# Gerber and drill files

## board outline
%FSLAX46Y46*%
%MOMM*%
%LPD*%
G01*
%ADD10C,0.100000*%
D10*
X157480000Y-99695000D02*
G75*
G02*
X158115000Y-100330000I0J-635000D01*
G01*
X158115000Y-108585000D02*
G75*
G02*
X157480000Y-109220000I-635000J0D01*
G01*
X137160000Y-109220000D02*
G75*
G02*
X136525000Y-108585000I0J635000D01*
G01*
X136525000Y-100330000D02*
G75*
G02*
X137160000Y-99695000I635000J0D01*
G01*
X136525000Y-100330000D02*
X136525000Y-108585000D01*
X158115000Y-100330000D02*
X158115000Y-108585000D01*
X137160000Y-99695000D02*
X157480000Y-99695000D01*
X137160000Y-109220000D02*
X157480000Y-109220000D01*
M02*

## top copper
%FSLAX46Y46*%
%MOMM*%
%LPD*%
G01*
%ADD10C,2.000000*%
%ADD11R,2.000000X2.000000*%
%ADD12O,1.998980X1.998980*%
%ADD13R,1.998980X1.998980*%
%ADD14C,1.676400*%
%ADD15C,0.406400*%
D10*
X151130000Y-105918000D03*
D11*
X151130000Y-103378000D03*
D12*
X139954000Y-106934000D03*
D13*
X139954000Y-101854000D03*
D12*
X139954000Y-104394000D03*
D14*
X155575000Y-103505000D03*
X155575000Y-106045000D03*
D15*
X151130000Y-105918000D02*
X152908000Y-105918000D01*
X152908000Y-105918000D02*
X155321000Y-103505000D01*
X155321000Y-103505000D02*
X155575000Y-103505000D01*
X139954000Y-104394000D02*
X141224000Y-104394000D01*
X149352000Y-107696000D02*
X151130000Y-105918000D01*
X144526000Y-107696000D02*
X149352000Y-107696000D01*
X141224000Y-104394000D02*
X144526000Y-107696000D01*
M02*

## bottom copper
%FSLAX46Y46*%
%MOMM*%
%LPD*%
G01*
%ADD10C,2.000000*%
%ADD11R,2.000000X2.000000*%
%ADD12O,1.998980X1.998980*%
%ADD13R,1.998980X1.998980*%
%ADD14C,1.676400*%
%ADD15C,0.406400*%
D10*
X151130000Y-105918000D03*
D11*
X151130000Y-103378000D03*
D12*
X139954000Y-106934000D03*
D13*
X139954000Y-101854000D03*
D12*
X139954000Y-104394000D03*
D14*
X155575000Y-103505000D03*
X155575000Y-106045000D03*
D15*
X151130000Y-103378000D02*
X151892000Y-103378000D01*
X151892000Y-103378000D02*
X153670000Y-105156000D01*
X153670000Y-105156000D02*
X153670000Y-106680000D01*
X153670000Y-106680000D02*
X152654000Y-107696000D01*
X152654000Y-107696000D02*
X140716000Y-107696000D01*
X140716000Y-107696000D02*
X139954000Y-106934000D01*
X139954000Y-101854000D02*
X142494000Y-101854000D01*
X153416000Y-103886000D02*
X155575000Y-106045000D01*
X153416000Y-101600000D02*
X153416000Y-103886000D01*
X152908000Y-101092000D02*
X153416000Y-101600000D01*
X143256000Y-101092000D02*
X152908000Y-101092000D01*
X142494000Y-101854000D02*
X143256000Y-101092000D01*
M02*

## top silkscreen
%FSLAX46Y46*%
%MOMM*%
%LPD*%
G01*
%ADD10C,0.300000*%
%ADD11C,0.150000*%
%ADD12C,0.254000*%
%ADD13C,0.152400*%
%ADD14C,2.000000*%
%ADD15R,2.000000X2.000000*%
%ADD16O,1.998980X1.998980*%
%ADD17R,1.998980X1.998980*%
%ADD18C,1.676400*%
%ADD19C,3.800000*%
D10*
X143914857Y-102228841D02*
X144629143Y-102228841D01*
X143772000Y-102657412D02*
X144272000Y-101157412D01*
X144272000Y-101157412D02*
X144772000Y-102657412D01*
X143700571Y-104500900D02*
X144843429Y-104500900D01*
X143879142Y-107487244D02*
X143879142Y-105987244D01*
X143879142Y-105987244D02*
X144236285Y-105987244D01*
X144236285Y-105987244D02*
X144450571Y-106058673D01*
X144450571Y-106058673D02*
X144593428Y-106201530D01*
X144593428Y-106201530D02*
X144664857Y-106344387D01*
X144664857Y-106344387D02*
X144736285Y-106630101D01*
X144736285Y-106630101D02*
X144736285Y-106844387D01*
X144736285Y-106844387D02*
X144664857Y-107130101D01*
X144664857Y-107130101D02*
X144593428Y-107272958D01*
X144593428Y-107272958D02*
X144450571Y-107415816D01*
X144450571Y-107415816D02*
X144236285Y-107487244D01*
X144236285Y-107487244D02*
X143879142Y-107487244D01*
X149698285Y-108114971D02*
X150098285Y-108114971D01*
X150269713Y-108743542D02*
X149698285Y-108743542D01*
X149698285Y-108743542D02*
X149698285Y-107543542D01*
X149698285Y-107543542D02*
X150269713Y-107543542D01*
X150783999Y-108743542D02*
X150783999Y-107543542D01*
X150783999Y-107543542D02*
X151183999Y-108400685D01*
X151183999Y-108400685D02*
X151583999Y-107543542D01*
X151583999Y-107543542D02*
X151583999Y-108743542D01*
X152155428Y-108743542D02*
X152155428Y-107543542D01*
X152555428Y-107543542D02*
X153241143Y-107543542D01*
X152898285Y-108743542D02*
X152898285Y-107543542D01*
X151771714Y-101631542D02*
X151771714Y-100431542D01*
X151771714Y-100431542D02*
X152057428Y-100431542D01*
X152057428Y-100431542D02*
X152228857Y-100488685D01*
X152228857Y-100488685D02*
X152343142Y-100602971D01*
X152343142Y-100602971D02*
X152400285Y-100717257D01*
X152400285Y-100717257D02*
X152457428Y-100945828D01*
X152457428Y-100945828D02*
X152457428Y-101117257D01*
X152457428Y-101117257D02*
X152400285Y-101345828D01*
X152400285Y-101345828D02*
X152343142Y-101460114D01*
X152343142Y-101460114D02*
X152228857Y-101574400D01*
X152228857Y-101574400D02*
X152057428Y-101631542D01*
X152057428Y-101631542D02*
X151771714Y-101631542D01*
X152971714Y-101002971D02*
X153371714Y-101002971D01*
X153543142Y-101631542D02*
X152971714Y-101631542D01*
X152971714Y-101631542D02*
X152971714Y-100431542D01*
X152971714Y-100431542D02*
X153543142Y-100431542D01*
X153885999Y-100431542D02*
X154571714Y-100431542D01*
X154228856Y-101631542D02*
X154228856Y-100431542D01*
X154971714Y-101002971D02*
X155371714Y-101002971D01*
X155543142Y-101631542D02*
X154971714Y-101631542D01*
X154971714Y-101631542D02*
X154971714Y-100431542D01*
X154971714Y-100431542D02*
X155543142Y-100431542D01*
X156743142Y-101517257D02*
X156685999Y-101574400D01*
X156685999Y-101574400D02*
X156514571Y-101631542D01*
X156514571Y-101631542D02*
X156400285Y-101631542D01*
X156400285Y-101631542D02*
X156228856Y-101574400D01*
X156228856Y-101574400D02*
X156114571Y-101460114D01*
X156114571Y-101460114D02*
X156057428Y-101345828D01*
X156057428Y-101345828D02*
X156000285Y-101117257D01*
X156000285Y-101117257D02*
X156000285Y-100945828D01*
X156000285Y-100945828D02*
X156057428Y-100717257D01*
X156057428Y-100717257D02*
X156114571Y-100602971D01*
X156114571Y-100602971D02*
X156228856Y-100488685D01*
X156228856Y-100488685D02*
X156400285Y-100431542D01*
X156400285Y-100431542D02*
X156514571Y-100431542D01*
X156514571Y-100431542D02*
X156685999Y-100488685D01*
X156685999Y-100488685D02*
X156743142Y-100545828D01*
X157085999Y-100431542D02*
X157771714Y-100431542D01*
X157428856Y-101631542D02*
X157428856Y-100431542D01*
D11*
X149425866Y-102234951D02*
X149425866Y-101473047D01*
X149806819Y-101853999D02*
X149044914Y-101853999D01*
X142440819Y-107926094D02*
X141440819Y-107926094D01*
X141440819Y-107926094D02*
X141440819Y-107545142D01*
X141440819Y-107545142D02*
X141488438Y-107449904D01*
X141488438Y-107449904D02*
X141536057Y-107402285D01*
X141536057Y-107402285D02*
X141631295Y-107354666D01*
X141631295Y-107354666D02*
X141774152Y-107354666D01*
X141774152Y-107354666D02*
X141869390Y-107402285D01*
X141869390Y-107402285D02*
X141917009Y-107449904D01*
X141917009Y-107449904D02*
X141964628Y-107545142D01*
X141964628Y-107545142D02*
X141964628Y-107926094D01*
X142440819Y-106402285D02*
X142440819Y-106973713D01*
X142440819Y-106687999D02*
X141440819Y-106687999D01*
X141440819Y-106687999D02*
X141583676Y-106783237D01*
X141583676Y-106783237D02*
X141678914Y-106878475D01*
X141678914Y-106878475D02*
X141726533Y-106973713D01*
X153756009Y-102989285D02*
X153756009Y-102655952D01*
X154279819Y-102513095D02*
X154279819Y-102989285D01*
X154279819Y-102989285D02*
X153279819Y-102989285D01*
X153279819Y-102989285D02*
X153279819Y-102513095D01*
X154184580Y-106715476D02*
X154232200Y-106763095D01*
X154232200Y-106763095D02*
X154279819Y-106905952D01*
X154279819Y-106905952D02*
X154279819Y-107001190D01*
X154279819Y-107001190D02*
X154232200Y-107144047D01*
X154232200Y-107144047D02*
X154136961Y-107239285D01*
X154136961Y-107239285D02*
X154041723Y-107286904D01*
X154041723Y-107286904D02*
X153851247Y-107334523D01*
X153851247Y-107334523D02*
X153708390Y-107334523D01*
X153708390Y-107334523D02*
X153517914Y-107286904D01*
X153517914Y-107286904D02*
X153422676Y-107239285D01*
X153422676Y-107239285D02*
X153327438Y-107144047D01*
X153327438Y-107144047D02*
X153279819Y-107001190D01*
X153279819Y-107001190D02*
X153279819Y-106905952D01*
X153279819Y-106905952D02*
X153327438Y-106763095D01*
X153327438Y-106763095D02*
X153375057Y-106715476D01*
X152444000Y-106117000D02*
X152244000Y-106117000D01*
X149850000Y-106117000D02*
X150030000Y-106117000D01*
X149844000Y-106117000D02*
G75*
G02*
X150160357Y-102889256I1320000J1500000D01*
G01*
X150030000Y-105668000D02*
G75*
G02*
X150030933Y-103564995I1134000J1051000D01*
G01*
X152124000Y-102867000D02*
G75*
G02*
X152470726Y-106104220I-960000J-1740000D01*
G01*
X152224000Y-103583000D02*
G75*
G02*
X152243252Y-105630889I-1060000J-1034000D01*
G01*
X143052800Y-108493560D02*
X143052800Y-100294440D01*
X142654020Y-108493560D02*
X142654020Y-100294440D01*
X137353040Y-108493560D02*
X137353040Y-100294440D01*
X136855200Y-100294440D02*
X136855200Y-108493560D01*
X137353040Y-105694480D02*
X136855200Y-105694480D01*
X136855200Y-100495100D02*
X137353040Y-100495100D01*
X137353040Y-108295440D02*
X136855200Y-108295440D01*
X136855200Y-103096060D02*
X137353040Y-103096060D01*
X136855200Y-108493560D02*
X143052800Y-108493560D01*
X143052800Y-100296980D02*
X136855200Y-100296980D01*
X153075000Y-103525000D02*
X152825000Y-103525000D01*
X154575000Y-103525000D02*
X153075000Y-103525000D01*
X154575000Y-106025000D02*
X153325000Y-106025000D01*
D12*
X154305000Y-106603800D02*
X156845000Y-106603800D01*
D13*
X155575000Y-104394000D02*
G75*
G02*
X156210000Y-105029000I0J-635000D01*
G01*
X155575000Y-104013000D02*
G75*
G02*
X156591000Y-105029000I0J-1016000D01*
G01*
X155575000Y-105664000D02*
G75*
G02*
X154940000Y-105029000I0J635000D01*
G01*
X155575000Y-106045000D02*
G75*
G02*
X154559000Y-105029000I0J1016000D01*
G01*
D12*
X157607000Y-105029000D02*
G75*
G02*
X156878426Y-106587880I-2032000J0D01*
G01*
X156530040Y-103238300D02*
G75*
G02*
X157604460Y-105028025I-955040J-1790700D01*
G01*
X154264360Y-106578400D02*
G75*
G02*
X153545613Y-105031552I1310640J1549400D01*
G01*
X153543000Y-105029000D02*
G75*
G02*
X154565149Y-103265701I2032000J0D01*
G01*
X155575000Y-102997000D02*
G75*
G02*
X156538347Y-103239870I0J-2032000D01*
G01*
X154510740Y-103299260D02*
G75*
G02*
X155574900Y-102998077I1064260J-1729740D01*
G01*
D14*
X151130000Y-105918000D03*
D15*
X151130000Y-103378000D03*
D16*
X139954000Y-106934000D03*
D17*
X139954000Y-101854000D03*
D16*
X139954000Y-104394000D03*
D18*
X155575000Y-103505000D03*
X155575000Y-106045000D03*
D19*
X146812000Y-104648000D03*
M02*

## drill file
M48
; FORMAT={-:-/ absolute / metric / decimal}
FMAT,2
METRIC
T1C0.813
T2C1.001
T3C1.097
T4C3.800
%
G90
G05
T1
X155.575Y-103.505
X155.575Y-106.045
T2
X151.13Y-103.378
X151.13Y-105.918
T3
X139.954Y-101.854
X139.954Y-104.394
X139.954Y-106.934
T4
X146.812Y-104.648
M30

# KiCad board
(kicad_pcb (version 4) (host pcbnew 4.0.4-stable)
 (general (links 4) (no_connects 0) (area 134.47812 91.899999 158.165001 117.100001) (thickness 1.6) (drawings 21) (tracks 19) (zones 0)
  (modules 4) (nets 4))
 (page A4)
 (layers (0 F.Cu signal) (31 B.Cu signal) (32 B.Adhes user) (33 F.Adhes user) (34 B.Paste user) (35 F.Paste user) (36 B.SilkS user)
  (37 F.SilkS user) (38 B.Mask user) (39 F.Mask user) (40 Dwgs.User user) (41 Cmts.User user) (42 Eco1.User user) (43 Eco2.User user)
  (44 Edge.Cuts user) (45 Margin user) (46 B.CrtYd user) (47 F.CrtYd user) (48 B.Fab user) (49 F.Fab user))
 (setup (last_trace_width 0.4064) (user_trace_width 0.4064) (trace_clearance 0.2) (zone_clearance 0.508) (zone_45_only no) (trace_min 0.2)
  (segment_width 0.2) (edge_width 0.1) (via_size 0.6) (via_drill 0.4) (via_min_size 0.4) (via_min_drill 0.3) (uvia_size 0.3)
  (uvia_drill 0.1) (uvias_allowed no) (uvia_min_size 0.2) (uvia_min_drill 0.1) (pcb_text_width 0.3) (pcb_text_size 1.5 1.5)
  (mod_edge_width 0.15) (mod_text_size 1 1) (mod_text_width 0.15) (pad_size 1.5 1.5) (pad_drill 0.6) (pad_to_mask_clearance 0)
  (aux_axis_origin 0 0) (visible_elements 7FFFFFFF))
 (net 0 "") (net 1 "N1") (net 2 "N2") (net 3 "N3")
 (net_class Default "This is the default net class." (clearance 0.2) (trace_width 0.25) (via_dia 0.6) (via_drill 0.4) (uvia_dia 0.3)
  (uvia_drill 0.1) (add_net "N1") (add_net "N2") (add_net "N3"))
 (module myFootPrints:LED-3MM (layer F.Cu) (at 151.13 105.918 90)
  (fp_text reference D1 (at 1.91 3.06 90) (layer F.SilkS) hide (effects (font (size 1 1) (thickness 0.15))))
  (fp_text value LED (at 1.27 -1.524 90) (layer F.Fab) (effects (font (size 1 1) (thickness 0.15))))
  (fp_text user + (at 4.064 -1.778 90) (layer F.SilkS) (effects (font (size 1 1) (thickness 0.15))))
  (fp_line (start -0.199 1.314) (end -0.199 1.114) (layer F.SilkS) (width 0.15))
  (fp_line (start -0.199 -1.28) (end -0.199 -1.1) (layer F.SilkS) (width 0.15))
  (fp_arc (start 1.301 0.034) (end -0.199 -1.286) (angle 108.5) (layer F.SilkS) (width 0.15))
  (fp_arc (start 1.301 0.034) (end 0.25 -1.1) (angle 85.7) (layer F.SilkS) (width 0.15))
  (fp_arc (start 1.311 0.034) (end 3.051 0.994) (angle 110) (layer F.SilkS) (width 0.15))
  (fp_arc (start 1.301 0.034) (end 2.335 1.094) (angle 87.5) (layer F.SilkS) (width 0.15))
  (pad 1 thru_hole circle (at 0 0 180) (size 2 2) (drill 1.00076) (layers *.Cu *.Mask F.SilkS) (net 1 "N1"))
  (pad 2 thru_hole rect (at 2.54 0 90) (size 2 2) (drill 1.00076) (layers *.Cu *.Mask F.SilkS) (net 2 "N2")))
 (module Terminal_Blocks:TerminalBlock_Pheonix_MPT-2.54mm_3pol (layer F.Cu) (at 139.954 101.854 270)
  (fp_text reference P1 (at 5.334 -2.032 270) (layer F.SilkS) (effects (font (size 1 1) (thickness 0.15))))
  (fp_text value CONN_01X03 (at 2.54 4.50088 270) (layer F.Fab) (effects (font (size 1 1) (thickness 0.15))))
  (fp_line (start 6.63956 -3.0988) (end -1.55956 -3.0988) (layer F.SilkS) (width 0.15))
  (fp_line (start 6.63956 -2.70002) (end -1.55956 -2.70002) (layer F.SilkS) (width 0.15))
  (fp_line (start 6.63956 2.60096) (end -1.55956 2.60096) (layer F.SilkS) (width 0.15))
  (fp_line (start -1.55956 3.0988) (end 6.63956 3.0988) (layer F.SilkS) (width 0.15))
  (fp_line (start 3.84048 2.60096) (end 3.84048 3.0988) (layer F.SilkS) (width 0.15))
  (fp_line (start -1.3589 3.0988) (end -1.3589 2.60096) (layer F.SilkS) (width 0.15))
  (fp_line (start 6.44144 2.60096) (end 6.44144 3.0988) (layer F.SilkS) (width 0.15))
  (fp_line (start 1.24206 3.0988) (end 1.24206 2.60096) (layer F.SilkS) (width 0.15))
  (fp_line (start 6.63956 3.0988) (end 6.63956 -3.0988) (layer F.SilkS) (width 0.15))
  (fp_line (start -1.55702 -3.0988) (end -1.55702 3.0988) (layer F.SilkS) (width 0.15))
  (pad 3 thru_hole oval (at 5.08 0 270) (size 1.99898 1.99898) (drill 1.09728) (layers *.Cu *.Mask F.SilkS) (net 2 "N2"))
  (pad 1 thru_hole rect (at 0 0 270) (size 1.99898 1.99898) (drill 1.09728) (layers *.Cu *.Mask F.SilkS) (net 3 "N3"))
  (pad 2 thru_hole oval (at 2.54 0 270) (size 1.99898 1.99898) (drill 1.09728) (layers *.Cu *.Mask F.SilkS) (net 1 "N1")))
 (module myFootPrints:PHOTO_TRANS (layer F.Cu) (at 155.575 104.775 270)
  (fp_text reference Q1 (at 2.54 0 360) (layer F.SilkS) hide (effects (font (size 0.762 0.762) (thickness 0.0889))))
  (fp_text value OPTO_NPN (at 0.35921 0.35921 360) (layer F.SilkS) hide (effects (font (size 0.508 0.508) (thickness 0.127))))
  (fp_line (start -1.25 2.5) (end -1.25 2.75) (layer F.SilkS) (width 0.15))
  (fp_line (start -1.25 1) (end -1.25 2.5) (layer F.SilkS) (width 0.15))
  (fp_line (start 1.25 1) (end 1.25 2.25) (layer F.SilkS) (width 0.15))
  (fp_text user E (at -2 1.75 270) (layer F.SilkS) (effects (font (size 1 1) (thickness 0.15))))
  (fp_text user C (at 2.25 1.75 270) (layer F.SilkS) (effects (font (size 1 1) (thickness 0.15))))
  (fp_line (start 1.8288 1.27) (end 1.8288 -1.27) (layer F.SilkS) (width 0.254))
  (fp_arc (start 0.254 0) (end -0.381 0) (angle 90) (layer F.SilkS) (width 0.1524))
  (fp_arc (start 0.254 0) (end -0.762 0) (angle 90) (layer F.SilkS) (width 0.1524))
  (fp_arc (start 0.254 0) (end 0.889 0) (angle 90) (layer F.SilkS) (width 0.1524))
  (fp_arc (start 0.254 0) (end 1.27 0) (angle 90) (layer F.SilkS) (width 0.1524))
  (fp_arc (start 0.254 0) (end 0.254 -2.032) (angle 50.1) (layer F.SilkS) (width 0.254))
  (fp_arc (start 0.254 0) (end -1.5367 -0.95504) (angle 61.9) (layer F.SilkS) (width 0.254))
  (fp_arc (start 0.254 0) (end 1.8034 1.31064) (angle 49.7) (layer F.SilkS) (width 0.254))
  (fp_arc (start 0.254 0) (end 0.254 2.032) (angle 60.2) (layer F.SilkS) (width 0.254))
  (fp_arc (start 0.254 0) (end -1.778 0) (angle 28.3) (layer F.SilkS) (width 0.254))
  (fp_arc (start 0.254 0) (end -1.47574 1.06426) (angle 31.6) (layer F.SilkS) (width 0.254))
  (pad 1 thru_hole circle (at -1.27 0 270) (size 1.6764 1.6764) (drill 0.8128) (layers *.Cu *.Mask F.SilkS) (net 1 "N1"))
  (pad 3 thru_hole circle (at 1.27 0 315) (size 1.6764 1.6764) (drill 0.8128) (layers *.Cu *.Mask F.SilkS) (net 3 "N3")))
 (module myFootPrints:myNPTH (layer F.Cu) (at 146.812 104.648)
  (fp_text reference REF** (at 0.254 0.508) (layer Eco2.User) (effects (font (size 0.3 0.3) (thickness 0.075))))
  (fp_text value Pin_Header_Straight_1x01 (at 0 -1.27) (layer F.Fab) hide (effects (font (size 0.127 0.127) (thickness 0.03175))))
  (pad "" np_thru_hole circle (at 0 0) (size 3.8 3.8) (drill 3.8) (layers *.Cu *.Mask F.SilkS) (thermal_width 4) (thermal_gap 4)))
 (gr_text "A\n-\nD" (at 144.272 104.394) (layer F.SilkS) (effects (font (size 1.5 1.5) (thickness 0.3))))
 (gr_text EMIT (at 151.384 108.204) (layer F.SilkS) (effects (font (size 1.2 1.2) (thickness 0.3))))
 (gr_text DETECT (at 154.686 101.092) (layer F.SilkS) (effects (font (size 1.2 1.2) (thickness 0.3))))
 (gr_arc (start 157.48 100.33) (end 157.48 99.695) (angle 90) (layer Edge.Cuts) (width 0.1))
 (gr_arc (start 157.48 108.585) (end 158.115 108.585) (angle 90) (layer Edge.Cuts) (width 0.1))
 (gr_arc (start 137.16 108.585) (end 137.16 109.22) (angle 90) (layer Edge.Cuts) (width 0.1))
 (gr_arc (start 137.16 100.33) (end 136.525 100.33) (angle 90) (layer Edge.Cuts) (width 0.1))
 (gr_line (start 136.525 100.33) (end 136.525 108.585) (angle 90) (layer Edge.Cuts) (width 0.1))
 (gr_line (start 158.115 100.33) (end 158.115 108.585) (angle 90) (layer Edge.Cuts) (width 0.1))
 (gr_line (start 137.16 99.695) (end 157.48 99.695) (angle 90) (layer Edge.Cuts) (width 0.1))
 (gr_line (start 137.16 109.22) (end 157.48 109.22) (angle 90) (layer Edge.Cuts) (width 0.1))
 (segment (start 151.13 105.918) (end 152.908 105.918) (width 0.4064) (layer F.Cu) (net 1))
 (segment (start 152.908 105.918) (end 155.321 103.505) (width 0.4064) (layer F.Cu) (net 1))
 (segment (start 155.321 103.505) (end 155.575 103.505) (width 0.4064) (layer F.Cu) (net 1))
 (segment (start 139.954 104.394) (end 141.224 104.394) (width 0.4064) (layer F.Cu) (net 1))
 (segment (start 149.352 107.696) (end 151.13 105.918) (width 0.4064) (layer F.Cu) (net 1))
 (segment (start 144.526 107.696) (end 149.352 107.696) (width 0.4064) (layer F.Cu) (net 1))
 (segment (start 141.224 104.394) (end 144.526 107.696) (width 0.4064) (layer F.Cu) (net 1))
 (segment (start 151.13 103.378) (end 151.892 103.378) (width 0.4064) (layer B.Cu) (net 2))
 (segment (start 151.892 103.378) (end 153.67 105.156) (width 0.4064) (layer B.Cu) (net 2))
 (segment (start 153.67 105.156) (end 153.67 106.68) (width 0.4064) (layer B.Cu) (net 2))
 (segment (start 153.67 106.68) (end 152.654 107.696) (width 0.4064) (layer B.Cu) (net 2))
 (segment (start 152.654 107.696) (end 140.716 107.696) (width 0.4064) (layer B.Cu) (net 2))
 (segment (start 140.716 107.696) (end 139.954 106.934) (width 0.4064) (layer B.Cu) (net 2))
 (segment (start 139.954 101.854) (end 142.494 101.854) (width 0.4064) (layer B.Cu) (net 3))
 (segment (start 153.416 103.886) (end 155.575 106.045) (width 0.4064) (layer B.Cu) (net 3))
 (segment (start 153.416 101.6) (end 153.416 103.886) (width 0.4064) (layer B.Cu) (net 3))
 (segment (start 152.908 101.092) (end 153.416 101.6) (width 0.4064) (layer B.Cu) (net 3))
 (segment (start 143.256 101.092) (end 152.908 101.092) (width 0.4064) (layer B.Cu) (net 3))
 (segment (start 142.494 101.854) (end 143.256 101.092) (width 0.4064) (layer B.Cu) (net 3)))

